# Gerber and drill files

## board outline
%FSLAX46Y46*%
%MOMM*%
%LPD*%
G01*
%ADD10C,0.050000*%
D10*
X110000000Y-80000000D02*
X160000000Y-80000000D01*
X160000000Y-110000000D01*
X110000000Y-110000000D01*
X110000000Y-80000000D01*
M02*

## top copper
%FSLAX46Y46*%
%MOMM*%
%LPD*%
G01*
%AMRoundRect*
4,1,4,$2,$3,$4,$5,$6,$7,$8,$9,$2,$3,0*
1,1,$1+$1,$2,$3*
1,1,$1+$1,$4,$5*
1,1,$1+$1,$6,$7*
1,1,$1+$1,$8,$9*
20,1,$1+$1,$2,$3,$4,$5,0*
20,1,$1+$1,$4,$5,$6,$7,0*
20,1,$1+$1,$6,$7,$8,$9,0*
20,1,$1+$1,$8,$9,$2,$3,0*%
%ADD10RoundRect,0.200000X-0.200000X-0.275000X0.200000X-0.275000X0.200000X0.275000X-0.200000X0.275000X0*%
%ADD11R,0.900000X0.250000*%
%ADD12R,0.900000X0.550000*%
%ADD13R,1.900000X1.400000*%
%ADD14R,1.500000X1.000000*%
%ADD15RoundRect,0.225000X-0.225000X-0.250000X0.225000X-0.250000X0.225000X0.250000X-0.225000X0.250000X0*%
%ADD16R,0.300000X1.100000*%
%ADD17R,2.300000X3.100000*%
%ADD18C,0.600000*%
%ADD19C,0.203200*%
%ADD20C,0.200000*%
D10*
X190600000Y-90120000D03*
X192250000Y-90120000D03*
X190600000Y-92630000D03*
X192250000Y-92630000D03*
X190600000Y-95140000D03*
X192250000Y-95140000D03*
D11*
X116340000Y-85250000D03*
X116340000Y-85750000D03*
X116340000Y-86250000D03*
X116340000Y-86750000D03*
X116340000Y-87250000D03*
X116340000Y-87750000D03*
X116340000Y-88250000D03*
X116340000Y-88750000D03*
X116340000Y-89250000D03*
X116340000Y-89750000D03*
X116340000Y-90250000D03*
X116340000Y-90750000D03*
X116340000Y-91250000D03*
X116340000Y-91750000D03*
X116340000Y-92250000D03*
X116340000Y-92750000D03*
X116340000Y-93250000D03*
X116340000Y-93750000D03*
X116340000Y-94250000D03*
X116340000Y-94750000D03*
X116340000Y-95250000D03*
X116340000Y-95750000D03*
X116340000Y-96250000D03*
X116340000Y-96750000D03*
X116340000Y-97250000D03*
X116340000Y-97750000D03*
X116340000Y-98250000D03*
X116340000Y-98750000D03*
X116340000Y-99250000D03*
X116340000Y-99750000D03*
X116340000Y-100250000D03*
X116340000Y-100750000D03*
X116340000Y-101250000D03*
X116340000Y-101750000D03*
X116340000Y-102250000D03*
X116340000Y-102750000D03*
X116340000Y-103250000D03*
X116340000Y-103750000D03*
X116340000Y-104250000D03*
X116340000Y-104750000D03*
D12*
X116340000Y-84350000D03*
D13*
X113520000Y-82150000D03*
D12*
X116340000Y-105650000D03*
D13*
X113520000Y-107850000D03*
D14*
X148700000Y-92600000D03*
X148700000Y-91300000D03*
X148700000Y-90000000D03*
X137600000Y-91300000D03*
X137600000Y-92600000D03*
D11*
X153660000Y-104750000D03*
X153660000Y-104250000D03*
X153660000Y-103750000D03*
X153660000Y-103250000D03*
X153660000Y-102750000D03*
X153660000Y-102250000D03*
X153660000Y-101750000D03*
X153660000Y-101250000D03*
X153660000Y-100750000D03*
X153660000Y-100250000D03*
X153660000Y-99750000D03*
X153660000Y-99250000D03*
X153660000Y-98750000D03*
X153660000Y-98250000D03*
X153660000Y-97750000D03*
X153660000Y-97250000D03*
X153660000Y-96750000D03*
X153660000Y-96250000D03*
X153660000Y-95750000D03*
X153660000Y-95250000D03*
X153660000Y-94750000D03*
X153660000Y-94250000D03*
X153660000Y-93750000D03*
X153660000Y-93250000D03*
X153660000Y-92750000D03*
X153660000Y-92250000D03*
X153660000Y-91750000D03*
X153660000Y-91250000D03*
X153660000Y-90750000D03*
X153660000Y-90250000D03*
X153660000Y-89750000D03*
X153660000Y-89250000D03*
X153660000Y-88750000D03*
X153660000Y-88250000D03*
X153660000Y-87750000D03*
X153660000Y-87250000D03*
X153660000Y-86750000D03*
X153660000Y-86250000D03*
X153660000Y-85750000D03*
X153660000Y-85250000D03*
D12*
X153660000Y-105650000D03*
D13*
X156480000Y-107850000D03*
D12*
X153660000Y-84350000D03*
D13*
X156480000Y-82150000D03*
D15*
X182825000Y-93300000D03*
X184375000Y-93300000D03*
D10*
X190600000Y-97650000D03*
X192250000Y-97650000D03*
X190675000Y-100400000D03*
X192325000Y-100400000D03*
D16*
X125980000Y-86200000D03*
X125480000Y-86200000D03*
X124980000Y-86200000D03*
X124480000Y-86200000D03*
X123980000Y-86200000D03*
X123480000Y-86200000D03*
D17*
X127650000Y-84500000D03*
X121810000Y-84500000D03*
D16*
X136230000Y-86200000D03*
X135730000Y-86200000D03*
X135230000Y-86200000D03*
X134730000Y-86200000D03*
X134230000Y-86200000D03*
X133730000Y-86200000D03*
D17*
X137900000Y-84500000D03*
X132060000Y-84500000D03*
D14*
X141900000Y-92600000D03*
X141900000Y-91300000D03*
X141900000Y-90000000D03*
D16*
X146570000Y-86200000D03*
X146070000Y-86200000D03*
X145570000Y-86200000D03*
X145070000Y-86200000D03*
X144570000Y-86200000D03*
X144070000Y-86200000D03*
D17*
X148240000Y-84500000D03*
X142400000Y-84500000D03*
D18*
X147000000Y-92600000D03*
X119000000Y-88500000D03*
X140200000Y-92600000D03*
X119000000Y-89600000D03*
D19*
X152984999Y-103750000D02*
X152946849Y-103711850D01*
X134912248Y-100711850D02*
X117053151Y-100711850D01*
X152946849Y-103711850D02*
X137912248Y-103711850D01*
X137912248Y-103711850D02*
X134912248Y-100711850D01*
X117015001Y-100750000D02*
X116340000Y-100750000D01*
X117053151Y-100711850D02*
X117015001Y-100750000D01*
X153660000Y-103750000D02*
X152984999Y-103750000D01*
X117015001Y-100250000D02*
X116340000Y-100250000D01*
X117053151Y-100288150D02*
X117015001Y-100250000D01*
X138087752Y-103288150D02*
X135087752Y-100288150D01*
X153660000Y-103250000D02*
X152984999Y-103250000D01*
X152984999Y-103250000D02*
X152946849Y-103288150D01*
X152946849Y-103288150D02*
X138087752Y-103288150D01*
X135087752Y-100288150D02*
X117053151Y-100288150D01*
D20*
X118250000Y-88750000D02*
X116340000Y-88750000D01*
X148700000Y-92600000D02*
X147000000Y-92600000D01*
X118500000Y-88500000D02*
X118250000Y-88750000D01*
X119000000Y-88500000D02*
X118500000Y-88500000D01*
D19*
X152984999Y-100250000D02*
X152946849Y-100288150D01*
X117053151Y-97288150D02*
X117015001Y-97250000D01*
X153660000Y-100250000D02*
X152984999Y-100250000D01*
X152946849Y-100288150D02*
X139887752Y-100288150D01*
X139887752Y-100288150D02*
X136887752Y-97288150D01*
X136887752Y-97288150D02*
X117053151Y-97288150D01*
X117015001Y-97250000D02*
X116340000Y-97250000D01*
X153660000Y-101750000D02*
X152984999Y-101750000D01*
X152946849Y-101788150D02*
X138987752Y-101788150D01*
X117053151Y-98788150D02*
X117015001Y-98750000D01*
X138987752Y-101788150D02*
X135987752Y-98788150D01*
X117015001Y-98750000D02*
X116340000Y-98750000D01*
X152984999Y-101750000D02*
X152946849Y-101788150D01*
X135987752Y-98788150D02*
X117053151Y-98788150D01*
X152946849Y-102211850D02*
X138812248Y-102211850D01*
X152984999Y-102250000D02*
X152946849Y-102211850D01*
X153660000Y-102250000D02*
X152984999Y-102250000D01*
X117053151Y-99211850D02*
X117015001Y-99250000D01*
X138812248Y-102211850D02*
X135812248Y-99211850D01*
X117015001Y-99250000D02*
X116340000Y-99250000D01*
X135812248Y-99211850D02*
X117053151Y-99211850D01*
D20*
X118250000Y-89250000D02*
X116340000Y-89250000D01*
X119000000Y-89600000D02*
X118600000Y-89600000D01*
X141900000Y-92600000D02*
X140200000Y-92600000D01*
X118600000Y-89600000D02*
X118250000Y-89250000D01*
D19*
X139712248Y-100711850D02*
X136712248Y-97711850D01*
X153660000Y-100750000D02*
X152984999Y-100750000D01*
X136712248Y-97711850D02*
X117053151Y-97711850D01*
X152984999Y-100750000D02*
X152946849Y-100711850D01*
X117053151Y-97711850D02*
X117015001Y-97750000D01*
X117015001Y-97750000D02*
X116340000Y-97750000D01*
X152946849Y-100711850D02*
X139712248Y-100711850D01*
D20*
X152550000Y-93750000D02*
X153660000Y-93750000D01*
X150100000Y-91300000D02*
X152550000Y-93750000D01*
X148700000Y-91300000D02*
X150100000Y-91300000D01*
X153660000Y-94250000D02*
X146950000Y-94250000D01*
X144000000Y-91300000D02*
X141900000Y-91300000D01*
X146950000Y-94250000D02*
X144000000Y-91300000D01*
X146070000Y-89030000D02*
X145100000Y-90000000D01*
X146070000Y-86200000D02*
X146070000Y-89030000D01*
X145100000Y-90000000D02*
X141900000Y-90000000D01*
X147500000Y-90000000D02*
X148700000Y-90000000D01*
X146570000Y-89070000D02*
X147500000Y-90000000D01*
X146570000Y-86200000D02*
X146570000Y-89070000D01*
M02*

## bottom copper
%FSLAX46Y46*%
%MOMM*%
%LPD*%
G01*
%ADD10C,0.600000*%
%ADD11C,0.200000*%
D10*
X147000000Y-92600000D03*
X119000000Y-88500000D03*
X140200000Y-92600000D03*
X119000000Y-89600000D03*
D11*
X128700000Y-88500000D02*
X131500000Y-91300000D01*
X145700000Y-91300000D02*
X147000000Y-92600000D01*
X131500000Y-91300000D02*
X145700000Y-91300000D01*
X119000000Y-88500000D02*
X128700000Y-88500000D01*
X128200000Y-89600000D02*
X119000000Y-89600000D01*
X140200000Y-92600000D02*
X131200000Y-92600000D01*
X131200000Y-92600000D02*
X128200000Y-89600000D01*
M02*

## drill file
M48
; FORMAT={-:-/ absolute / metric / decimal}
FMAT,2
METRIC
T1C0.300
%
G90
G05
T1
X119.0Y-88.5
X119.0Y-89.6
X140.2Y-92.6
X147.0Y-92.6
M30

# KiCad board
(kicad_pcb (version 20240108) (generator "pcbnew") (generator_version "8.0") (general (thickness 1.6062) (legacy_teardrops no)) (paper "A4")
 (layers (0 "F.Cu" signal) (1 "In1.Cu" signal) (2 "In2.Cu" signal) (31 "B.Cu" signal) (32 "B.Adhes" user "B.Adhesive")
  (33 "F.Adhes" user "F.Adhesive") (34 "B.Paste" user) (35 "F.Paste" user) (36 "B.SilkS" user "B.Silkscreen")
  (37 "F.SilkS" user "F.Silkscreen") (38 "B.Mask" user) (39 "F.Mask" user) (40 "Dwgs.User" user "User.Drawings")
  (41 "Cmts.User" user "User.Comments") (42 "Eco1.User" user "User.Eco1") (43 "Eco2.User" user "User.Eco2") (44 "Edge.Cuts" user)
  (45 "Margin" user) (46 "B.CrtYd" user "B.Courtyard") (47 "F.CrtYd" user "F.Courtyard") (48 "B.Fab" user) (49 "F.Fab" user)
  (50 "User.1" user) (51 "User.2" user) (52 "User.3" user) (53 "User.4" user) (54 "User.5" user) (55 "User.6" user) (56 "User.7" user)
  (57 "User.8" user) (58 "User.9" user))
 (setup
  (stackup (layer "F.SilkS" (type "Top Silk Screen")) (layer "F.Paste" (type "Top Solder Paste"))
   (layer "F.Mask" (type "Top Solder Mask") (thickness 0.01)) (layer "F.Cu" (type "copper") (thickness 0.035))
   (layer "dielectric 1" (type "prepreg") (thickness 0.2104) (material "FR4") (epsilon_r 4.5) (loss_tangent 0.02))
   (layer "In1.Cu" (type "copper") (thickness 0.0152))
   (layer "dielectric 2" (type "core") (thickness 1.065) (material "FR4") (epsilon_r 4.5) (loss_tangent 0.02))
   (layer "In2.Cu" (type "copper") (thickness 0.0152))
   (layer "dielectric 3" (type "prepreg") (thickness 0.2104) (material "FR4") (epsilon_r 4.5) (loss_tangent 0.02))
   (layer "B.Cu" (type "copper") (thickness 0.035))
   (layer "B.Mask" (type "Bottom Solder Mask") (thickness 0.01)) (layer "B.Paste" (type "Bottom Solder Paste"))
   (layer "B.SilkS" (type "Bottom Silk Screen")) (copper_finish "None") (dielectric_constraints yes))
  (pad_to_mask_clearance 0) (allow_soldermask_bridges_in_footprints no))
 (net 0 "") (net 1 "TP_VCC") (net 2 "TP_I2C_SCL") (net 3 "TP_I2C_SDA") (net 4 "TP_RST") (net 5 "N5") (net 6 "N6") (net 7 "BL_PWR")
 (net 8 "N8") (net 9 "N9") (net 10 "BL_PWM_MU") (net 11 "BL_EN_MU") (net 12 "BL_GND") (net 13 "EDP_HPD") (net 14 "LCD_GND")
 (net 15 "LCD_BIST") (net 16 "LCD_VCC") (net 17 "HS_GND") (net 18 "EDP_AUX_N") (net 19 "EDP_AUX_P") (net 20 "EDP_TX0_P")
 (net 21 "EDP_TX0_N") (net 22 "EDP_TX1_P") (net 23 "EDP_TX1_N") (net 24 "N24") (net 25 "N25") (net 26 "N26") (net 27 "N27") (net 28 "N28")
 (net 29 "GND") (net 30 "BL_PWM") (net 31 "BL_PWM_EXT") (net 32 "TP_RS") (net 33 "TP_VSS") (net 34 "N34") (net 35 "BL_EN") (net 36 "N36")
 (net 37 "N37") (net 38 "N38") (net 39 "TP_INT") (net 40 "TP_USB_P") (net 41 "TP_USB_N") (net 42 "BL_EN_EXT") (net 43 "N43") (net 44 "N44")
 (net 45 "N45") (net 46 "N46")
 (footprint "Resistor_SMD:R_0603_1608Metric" (layer "F.Cu") (at 191.425 90.12)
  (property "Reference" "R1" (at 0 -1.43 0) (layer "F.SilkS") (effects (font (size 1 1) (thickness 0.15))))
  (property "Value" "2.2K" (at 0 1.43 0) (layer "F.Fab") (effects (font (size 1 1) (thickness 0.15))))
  (pad "1" smd roundrect (at -0.825 0) (size 0.8 0.95) (layers "F.Cu" "F.Paste" "F.Mask") (roundrect_rratio 0.25) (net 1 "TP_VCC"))
  (pad "2" smd roundrect (at 0.825 0) (size 0.8 0.95) (layers "F.Cu" "F.Paste" "F.Mask") (roundrect_rratio 0.25) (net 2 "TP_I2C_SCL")))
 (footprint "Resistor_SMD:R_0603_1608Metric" (layer "F.Cu") (at 191.425 92.63)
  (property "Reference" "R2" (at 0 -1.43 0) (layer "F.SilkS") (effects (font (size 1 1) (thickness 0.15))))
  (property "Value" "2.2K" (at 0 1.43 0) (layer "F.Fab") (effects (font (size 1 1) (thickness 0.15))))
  (pad "1" smd roundrect (at -0.825 0) (size 0.8 0.95) (layers "F.Cu" "F.Paste" "F.Mask") (roundrect_rratio 0.25) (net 1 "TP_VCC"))
  (pad "2" smd roundrect (at 0.825 0) (size 0.8 0.95) (layers "F.Cu" "F.Paste" "F.Mask") (roundrect_rratio 0.25) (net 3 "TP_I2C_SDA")))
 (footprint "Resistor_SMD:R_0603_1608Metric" (layer "F.Cu") (at 191.425 95.14)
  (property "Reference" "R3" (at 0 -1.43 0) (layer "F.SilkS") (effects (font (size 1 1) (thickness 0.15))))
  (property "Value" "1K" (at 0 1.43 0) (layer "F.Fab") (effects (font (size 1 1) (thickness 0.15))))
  (pad "1" smd roundrect (at -0.825 0) (size 0.8 0.95) (layers "F.Cu" "F.Paste" "F.Mask") (roundrect_rratio 0.25) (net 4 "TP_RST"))
  (pad "2" smd roundrect (at 0.825 0) (size 0.8 0.95) (layers "F.Cu" "F.Paste" "F.Mask") (roundrect_rratio 0.25) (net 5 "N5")))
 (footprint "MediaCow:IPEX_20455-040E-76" (layer "F.Cu") (at 114.42 95 -90)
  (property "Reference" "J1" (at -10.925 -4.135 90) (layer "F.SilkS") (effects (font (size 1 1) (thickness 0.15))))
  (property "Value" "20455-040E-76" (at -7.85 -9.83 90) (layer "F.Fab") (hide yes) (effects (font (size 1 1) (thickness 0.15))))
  (pad "1" smd rect (at -9.75 -1.92 270) (size 0.25 0.9) (layers "F.Cu" "F.Paste" "F.Mask") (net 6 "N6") (solder_mask_margin 0.102))
  (pad "2" smd rect (at -9.25 -1.92 270) (size 0.25 0.9) (layers "F.Cu" "F.Paste" "F.Mask") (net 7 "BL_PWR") (solder_mask_margin 0.102))
  (pad "3" smd rect (at -8.75 -1.92 270) (size 0.25 0.9) (layers "F.Cu" "F.Paste" "F.Mask") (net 7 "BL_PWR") (solder_mask_margin 0.102))
  (pad "4" smd rect (at -8.25 -1.92 270) (size 0.25 0.9) (layers "F.Cu" "F.Paste" "F.Mask") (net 7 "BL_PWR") (solder_mask_margin 0.102))
  (pad "5" smd rect (at -7.75 -1.92 270) (size 0.25 0.9) (layers "F.Cu" "F.Paste" "F.Mask") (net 7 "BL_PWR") (solder_mask_margin 0.102))
  (pad "6" smd rect (at -7.25 -1.92 270) (size 0.25 0.9) (layers "F.Cu" "F.Paste" "F.Mask") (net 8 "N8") (solder_mask_margin 0.102))
  (pad "7" smd rect (at -6.75 -1.92 270) (size 0.25 0.9) (layers "F.Cu" "F.Paste" "F.Mask") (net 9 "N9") (solder_mask_margin 0.102))
  (pad "8" smd rect (at -6.25 -1.92 270) (size 0.25 0.9) (layers "F.Cu" "F.Paste" "F.Mask") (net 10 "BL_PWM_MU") (solder_mask_margin 0.102))
  (pad "9" smd rect (at -5.75 -1.92 270) (size 0.25 0.9) (layers "F.Cu" "F.Paste" "F.Mask") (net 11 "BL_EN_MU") (solder_mask_margin 0.102))
  (pad "10" smd rect (at -5.25 -1.92 270) (size 0.25 0.9) (layers "F.Cu" "F.Paste" "F.Mask") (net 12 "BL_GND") (solder_mask_margin 0.102))
  (pad "11" smd rect (at -4.75 -1.92 270) (size 0.25 0.9) (layers "F.Cu" "F.Paste" "F.Mask") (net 12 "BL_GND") (solder_mask_margin 0.102))
  (pad "12" smd rect (at -4.25 -1.92 270) (size 0.25 0.9) (layers "F.Cu" "F.Paste" "F.Mask") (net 12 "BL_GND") (solder_mask_margin 0.102))
  (pad "13" smd rect (at -3.75 -1.92 270) (size 0.25 0.9) (layers "F.Cu" "F.Paste" "F.Mask") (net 12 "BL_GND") (solder_mask_margin 0.102))
  (pad "14" smd rect (at -3.25 -1.92 270) (size 0.25 0.9) (layers "F.Cu" "F.Paste" "F.Mask") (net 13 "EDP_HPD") (solder_mask_margin 0.102))
  (pad "15" smd rect (at -2.75 -1.92 270) (size 0.25 0.9) (layers "F.Cu" "F.Paste" "F.Mask") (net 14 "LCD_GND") (solder_mask_margin 0.102))
  (pad "16" smd rect (at -2.25 -1.92 270) (size 0.25 0.9) (layers "F.Cu" "F.Paste" "F.Mask") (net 14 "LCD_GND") (solder_mask_margin 0.102))
  (pad "17" smd rect (at -1.75 -1.92 270) (size 0.25 0.9) (layers "F.Cu" "F.Paste" "F.Mask") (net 14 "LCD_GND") (solder_mask_margin 0.102))
  (pad "18" smd rect (at -1.25 -1.92 270) (size 0.25 0.9) (layers "F.Cu" "F.Paste" "F.Mask") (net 14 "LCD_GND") (solder_mask_margin 0.102))
  (pad "19" smd rect (at -0.75 -1.92 270) (size 0.25 0.9) (layers "F.Cu" "F.Paste" "F.Mask") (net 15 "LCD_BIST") (solder_mask_margin 0.102))
  (pad "20" smd rect (at -0.25 -1.92 270) (size 0.25 0.9) (layers "F.Cu" "F.Paste" "F.Mask") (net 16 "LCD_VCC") (solder_mask_margin 0.102))
  (pad "21" smd rect (at 0.25 -1.92 270) (size 0.25 0.9) (layers "F.Cu" "F.Paste" "F.Mask") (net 16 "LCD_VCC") (solder_mask_margin 0.102))
  (pad "22" smd rect (at 0.75 -1.92 270) (size 0.25 0.9) (layers "F.Cu" "F.Paste" "F.Mask") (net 16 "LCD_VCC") (solder_mask_margin 0.102))
  (pad "23" smd rect (at 1.25 -1.92 270) (size 0.25 0.9) (layers "F.Cu" "F.Paste" "F.Mask") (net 16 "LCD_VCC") (solder_mask_margin 0.102))
  (pad "24" smd rect (at 1.75 -1.92 270) (size 0.25 0.9) (layers "F.Cu" "F.Paste" "F.Mask") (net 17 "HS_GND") (solder_mask_margin 0.102))
  (pad "25" smd rect (at 2.25 -1.92 270) (size 0.25 0.9) (layers "F.Cu" "F.Paste" "F.Mask") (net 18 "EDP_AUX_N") (solder_mask_margin 0.102))
  (pad "26" smd rect (at 2.75 -1.92 270) (size 0.25 0.9) (layers "F.Cu" "F.Paste" "F.Mask") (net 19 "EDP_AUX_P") (solder_mask_margin 0.102))
  (pad "27" smd rect (at 3.25 -1.92 270) (size 0.25 0.9) (layers "F.Cu" "F.Paste" "F.Mask") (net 17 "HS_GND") (solder_mask_margin 0.102))
  (pad "28" smd rect (at 3.75 -1.92 270) (size 0.25 0.9) (layers "F.Cu" "F.Paste" "F.Mask") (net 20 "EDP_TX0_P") (solder_mask_margin 0.102))
  (pad "29" smd rect (at 4.25 -1.92 270) (size 0.25 0.9) (layers "F.Cu" "F.Paste" "F.Mask") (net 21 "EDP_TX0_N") (solder_mask_margin 0.102))
  (pad "30" smd rect (at 4.75 -1.92 270) (size 0.25 0.9) (layers "F.Cu" "F.Paste" "F.Mask") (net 17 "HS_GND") (solder_mask_margin 0.102))
  (pad "31" smd rect (at 5.25 -1.92 270) (size 0.25 0.9) (layers "F.Cu" "F.Paste" "F.Mask") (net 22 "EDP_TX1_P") (solder_mask_margin 0.102))
  (pad "32" smd rect (at 5.75 -1.92 270) (size 0.25 0.9) (layers "F.Cu" "F.Paste" "F.Mask") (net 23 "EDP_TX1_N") (solder_mask_margin 0.102))
  (pad "33" smd rect (at 6.25 -1.92 270) (size 0.25 0.9) (layers "F.Cu" "F.Paste" "F.Mask") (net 17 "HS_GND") (solder_mask_margin 0.102))
  (pad "34" smd rect (at 6.75 -1.92 270) (size 0.25 0.9) (layers "F.Cu" "F.Paste" "F.Mask") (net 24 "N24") (solder_mask_margin 0.102))
  (pad "35" smd rect (at 7.25 -1.92 270) (size 0.25 0.9) (layers "F.Cu" "F.Paste" "F.Mask") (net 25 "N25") (solder_mask_margin 0.102))
  (pad "36" smd rect (at 7.75 -1.92 270) (size 0.25 0.9) (layers "F.Cu" "F.Paste" "F.Mask") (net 17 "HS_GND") (solder_mask_margin 0.102))
  (pad "37" smd rect (at 8.25 -1.92 270) (size 0.25 0.9) (layers "F.Cu" "F.Paste" "F.Mask") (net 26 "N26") (solder_mask_margin 0.102))
  (pad "38" smd rect (at 8.75 -1.92 270) (size 0.25 0.9) (layers "F.Cu" "F.Paste" "F.Mask") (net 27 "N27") (solder_mask_margin 0.102))
  (pad "39" smd rect (at 9.25 -1.92 270) (size 0.25 0.9) (layers "F.Cu" "F.Paste" "F.Mask") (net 17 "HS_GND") (solder_mask_margin 0.102))
  (pad "40" smd rect (at 9.75 -1.92 270) (size 0.25 0.9) (layers "F.Cu" "F.Paste" "F.Mask") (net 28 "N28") (solder_mask_margin 0.102))
  (pad "S1" smd rect (at -10.65 -1.92 270) (size 0.55 0.9) (layers "F.Cu" "F.Paste" "F.Mask") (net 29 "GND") (solder_mask_margin 0.102))
  (pad "S2" smd rect (at -12.85 0.9 270) (size 1.4 1.9) (layers "F.Cu" "F.Paste" "F.Mask") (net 29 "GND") (solder_mask_margin 0.102))
  (pad "S3" smd rect (at 10.65 -1.92 270) (size 0.55 0.9) (layers "F.Cu" "F.Paste" "F.Mask") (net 29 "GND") (solder_mask_margin 0.102))
  (pad "S4" smd rect (at 12.85 0.9 270) (size 1.4 1.9) (layers "F.Cu" "F.Paste" "F.Mask") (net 29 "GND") (solder_mask_margin 0.102)))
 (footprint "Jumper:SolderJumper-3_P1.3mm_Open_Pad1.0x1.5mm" (layer "F.Cu") (at 148.7 91.3 90)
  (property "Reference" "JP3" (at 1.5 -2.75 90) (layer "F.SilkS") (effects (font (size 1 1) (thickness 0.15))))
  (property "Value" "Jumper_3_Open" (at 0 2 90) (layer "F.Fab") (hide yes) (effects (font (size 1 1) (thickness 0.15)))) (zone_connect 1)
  (pad "1" smd rect (at -1.3 0 90) (size 1 1.5) (layers "F.Cu" "F.Mask") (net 10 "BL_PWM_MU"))
  (pad "2" smd rect (at 0 0 90) (size 1 1.5) (layers "F.Cu" "F.Mask") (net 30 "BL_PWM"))
  (pad "3" smd rect (at 1.3 0 90) (size 1 1.5) (layers "F.Cu" "F.Mask") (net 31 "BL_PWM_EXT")))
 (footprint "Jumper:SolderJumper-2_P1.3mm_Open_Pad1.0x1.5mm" (layer "F.Cu") (at 137.6 91.95 -90)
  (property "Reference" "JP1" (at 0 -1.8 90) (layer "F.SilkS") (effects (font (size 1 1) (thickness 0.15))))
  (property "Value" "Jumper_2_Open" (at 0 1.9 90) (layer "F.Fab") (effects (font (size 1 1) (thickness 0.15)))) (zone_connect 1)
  (pad "1" smd rect (at -0.65 0 270) (size 1 1.5) (layers "F.Cu" "F.Mask") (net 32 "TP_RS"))
  (pad "2" smd rect (at 0.65 0 270) (size 1 1.5) (layers "F.Cu" "F.Mask") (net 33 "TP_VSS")))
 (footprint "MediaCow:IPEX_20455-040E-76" (layer "F.Cu") (at 155.58 95 90)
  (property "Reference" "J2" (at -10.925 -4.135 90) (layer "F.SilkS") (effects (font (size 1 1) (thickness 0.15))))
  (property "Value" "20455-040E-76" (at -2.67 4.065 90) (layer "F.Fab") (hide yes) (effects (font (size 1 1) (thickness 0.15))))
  (pad "1" smd rect (at -9.75 -1.92 90) (size 0.25 0.9) (layers "F.Cu" "F.Paste" "F.Mask") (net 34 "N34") (solder_mask_margin 0.102))
  (pad "2" smd rect (at -9.25 -1.92 90) (size 0.25 0.9) (layers "F.Cu" "F.Paste" "F.Mask") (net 17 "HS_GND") (solder_mask_margin 0.102))
  (pad "3" smd rect (at -8.75 -1.92 90) (size 0.25 0.9) (layers "F.Cu" "F.Paste" "F.Mask") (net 23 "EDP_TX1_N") (solder_mask_margin 0.102))
  (pad "4" smd rect (at -8.25 -1.92 90) (size 0.25 0.9) (layers "F.Cu" "F.Paste" "F.Mask") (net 22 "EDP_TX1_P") (solder_mask_margin 0.102))
  (pad "5" smd rect (at -7.75 -1.92 90) (size 0.25 0.9) (layers "F.Cu" "F.Paste" "F.Mask") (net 17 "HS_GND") (solder_mask_margin 0.102))
  (pad "6" smd rect (at -7.25 -1.92 90) (size 0.25 0.9) (layers "F.Cu" "F.Paste" "F.Mask") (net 21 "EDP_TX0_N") (solder_mask_margin 0.102))
  (pad "7" smd rect (at -6.75 -1.92 90) (size 0.25 0.9) (layers "F.Cu" "F.Paste" "F.Mask") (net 20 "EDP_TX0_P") (solder_mask_margin 0.102))
  (pad "8" smd rect (at -6.25 -1.92 90) (size 0.25 0.9) (layers "F.Cu" "F.Paste" "F.Mask") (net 17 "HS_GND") (solder_mask_margin 0.102))
  (pad "9" smd rect (at -5.75 -1.92 90) (size 0.25 0.9) (layers "F.Cu" "F.Paste" "F.Mask") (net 19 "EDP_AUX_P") (solder_mask_margin 0.102))
  (pad "10" smd rect (at -5.25 -1.92 90) (size 0.25 0.9) (layers "F.Cu" "F.Paste" "F.Mask") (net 18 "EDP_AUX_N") (solder_mask_margin 0.102))
  (pad "11" smd rect (at -4.75 -1.92 90) (size 0.25 0.9) (layers "F.Cu" "F.Paste" "F.Mask") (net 17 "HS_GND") (solder_mask_margin 0.102))
  (pad "12" smd rect (at -4.25 -1.92 90) (size 0.25 0.9) (layers "F.Cu" "F.Paste" "F.Mask") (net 16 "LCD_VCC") (solder_mask_margin 0.102))
  (pad "13" smd rect (at -3.75 -1.92 90) (size 0.25 0.9) (layers "F.Cu" "F.Paste" "F.Mask") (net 16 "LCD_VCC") (solder_mask_margin 0.102))
  (pad "14" smd rect (at -3.25 -1.92 90) (size 0.25 0.9) (layers "F.Cu" "F.Paste" "F.Mask") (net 15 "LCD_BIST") (solder_mask_margin 0.102))
  (pad "15" smd rect (at -2.75 -1.92 90) (size 0.25 0.9) (layers "F.Cu" "F.Paste" "F.Mask") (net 14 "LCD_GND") (solder_mask_margin 0.102))
  (pad "16" smd rect (at -2.25 -1.92 90) (size 0.25 0.9) (layers "F.Cu" "F.Paste" "F.Mask") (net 14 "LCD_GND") (solder_mask_margin 0.102))
  (pad "17" smd rect (at -1.75 -1.92 90) (size 0.25 0.9) (layers "F.Cu" "F.Paste" "F.Mask") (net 13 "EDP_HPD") (solder_mask_margin 0.102))
  (pad "18" smd rect (at -1.25 -1.92 90) (size 0.25 0.9) (layers "F.Cu" "F.Paste" "F.Mask") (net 12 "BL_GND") (solder_mask_margin 0.102))
  (pad "19" smd rect (at -0.75 -1.92 90) (size 0.25 0.9) (layers "F.Cu" "F.Paste" "F.Mask") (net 12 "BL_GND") (solder_mask_margin 0.102))
  (pad "20" smd rect (at -0.25 -1.92 90) (size 0.25 0.9) (layers "F.Cu" "F.Paste" "F.Mask") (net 12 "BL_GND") (solder_mask_margin 0.102))
  (pad "21" smd rect (at 0.25 -1.92 90) (size 0.25 0.9) (layers "F.Cu" "F.Paste" "F.Mask") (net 12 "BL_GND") (solder_mask_margin 0.102))
  (pad "22" smd rect (at 0.75 -1.92 90) (size 0.25 0.9) (layers "F.Cu" "F.Paste" "F.Mask") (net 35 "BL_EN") (solder_mask_margin 0.102))
  (pad "23" smd rect (at 1.25 -1.92 90) (size 0.25 0.9) (layers "F.Cu" "F.Paste" "F.Mask") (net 30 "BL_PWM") (solder_mask_margin 0.102))
  (pad "24" smd rect (at 1.75 -1.92 90) (size 0.25 0.9) (layers "F.Cu" "F.Paste" "F.Mask") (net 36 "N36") (solder_mask_margin 0.102))
  (pad "25" smd rect (at 2.25 -1.92 90) (size 0.25 0.9) (layers "F.Cu" "F.Paste" "F.Mask") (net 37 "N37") (solder_mask_margin 0.102))
  (pad "26" smd rect (at 2.75 -1.92 90) (size 0.25 0.9) (layers "F.Cu" "F.Paste" "F.Mask") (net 7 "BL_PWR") (solder_mask_margin 0.102))
  (pad "27" smd rect (at 3.25 -1.92 90) (size 0.25 0.9) (layers "F.Cu" "F.Paste" "F.Mask") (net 7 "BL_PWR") (solder_mask_margin 0.102))
  (pad "28" smd rect (at 3.75 -1.92 90) (size 0.25 0.9) (layers "F.Cu" "F.Paste" "F.Mask") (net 7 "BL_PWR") (solder_mask_margin 0.102))
  (pad "29" smd rect (at 4.25 -1.92 90) (size 0.25 0.9) (layers "F.Cu" "F.Paste" "F.Mask") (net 7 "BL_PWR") (solder_mask_margin 0.102))
  (pad "30" smd rect (at 4.75 -1.92 90) (size 0.25 0.9) (layers "F.Cu" "F.Paste" "F.Mask") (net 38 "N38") (solder_mask_margin 0.102))
  (pad "31" smd rect (at 5.25 -1.92 90) (size 0.25 0.9) (layers "F.Cu" "F.Paste" "F.Mask") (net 4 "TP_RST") (solder_mask_margin 0.102))
  (pad "32" smd rect (at 5.75 -1.92 90) (size 0.25 0.9) (layers "F.Cu" "F.Paste" "F.Mask") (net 2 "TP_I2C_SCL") (solder_mask_margin 0.102))
  (pad "33" smd rect (at 6.25 -1.92 90) (size 0.25 0.9) (layers "F.Cu" "F.Paste" "F.Mask") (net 3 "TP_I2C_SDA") (solder_mask_margin 0.102))
  (pad "34" smd rect (at 6.75 -1.92 90) (size 0.25 0.9) (layers "F.Cu" "F.Paste" "F.Mask") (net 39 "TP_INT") (solder_mask_margin 0.102))
  (pad "35" smd rect (at 7.25 -1.92 90) (size 0.25 0.9) (layers "F.Cu" "F.Paste" "F.Mask") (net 33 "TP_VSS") (solder_mask_margin 0.102))
  (pad "36" smd rect (at 7.75 -1.92 90) (size 0.25 0.9) (layers "F.Cu" "F.Paste" "F.Mask") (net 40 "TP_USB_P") (solder_mask_margin 0.102))
  (pad "37" smd rect (at 8.25 -1.92 90) (size 0.25 0.9) (layers "F.Cu" "F.Paste" "F.Mask") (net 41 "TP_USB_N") (solder_mask_margin 0.102))
  (pad "38" smd rect (at 8.75 -1.92 90) (size 0.25 0.9) (layers "F.Cu" "F.Paste" "F.Mask") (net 33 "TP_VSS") (solder_mask_margin 0.102))
  (pad "39" smd rect (at 9.25 -1.92 90) (size 0.25 0.9) (layers "F.Cu" "F.Paste" "F.Mask") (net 32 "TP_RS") (solder_mask_margin 0.102))
  (pad "40" smd rect (at 9.75 -1.92 90) (size 0.25 0.9) (layers "F.Cu" "F.Paste" "F.Mask") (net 1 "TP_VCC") (solder_mask_margin 0.102))
  (pad "S1" smd rect (at -10.65 -1.92 90) (size 0.55 0.9) (layers "F.Cu" "F.Paste" "F.Mask") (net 29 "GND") (solder_mask_margin 0.102))
  (pad "S2" smd rect (at -12.85 0.9 90) (size 1.4 1.9) (layers "F.Cu" "F.Paste" "F.Mask") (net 29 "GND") (solder_mask_margin 0.102))
  (pad "S3" smd rect (at 10.65 -1.92 90) (size 0.55 0.9) (layers "F.Cu" "F.Paste" "F.Mask") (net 29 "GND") (solder_mask_margin 0.102))
  (pad "S4" smd rect (at 12.85 0.9 90) (size 1.4 1.9) (layers "F.Cu" "F.Paste" "F.Mask") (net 29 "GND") (solder_mask_margin 0.102)))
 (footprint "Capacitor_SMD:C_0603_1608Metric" (layer "F.Cu") (at 183.6 93.3)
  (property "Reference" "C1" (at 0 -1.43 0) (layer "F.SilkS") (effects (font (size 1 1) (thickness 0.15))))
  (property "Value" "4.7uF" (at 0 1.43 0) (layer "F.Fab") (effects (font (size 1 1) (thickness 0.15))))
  (pad "1" smd roundrect (at -0.775 0) (size 0.9 0.95) (layers "F.Cu" "F.Paste" "F.Mask") (roundrect_rratio 0.25) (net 5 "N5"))
  (pad "2" smd roundrect (at 0.775 0) (size 0.9 0.95) (layers "F.Cu" "F.Paste" "F.Mask") (roundrect_rratio 0.25) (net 33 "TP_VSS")))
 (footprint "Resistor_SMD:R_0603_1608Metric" (layer "F.Cu") (at 191.425 97.65)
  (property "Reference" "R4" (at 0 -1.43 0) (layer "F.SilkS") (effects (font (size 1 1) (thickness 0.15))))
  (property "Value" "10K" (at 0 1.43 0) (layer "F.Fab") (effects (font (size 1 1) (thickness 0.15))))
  (pad "1" smd roundrect (at -0.825 0) (size 0.8 0.95) (layers "F.Cu" "F.Paste" "F.Mask") (roundrect_rratio 0.25) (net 1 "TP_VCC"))
  (pad "2" smd roundrect (at 0.825 0) (size 0.8 0.95) (layers "F.Cu" "F.Paste" "F.Mask") (roundrect_rratio 0.25) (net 5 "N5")))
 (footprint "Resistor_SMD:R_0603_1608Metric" (layer "F.Cu") (at 191.5 100.4)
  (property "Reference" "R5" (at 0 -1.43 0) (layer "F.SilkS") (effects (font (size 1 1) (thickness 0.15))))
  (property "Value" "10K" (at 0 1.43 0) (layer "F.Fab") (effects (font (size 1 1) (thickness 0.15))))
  (pad "1" smd roundrect (at -0.825 0) (size 0.8 0.95) (layers "F.Cu" "F.Paste" "F.Mask") (roundrect_rratio 0.25) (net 1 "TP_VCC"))
  (pad "2" smd roundrect (at 0.825 0) (size 0.8 0.95) (layers "F.Cu" "F.Paste" "F.Mask") (roundrect_rratio 0.25) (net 32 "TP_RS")))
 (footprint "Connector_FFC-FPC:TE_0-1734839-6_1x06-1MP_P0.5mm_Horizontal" (layer "F.Cu") (at 124.73 84.85 180)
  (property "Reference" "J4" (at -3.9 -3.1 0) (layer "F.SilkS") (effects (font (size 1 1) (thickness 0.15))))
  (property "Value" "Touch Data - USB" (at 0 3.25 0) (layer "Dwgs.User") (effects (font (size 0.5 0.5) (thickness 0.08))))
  (pad "1" smd rect (at -1.25 -1.35 180) (size 0.3 1.1) (layers "F.Cu" "F.Paste" "F.Mask") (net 33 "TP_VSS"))
  (pad "2" smd rect (at -0.75 -1.35 180) (size 0.3 1.1) (layers "F.Cu" "F.Paste" "F.Mask") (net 40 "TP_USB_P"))
  (pad "3" smd rect (at -0.25 -1.35 180) (size 0.3 1.1) (layers "F.Cu" "F.Paste" "F.Mask") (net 41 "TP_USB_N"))
  (pad "4" smd rect (at 0.25 -1.35 180) (size 0.3 1.1) (layers "F.Cu" "F.Paste" "F.Mask") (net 33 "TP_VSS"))
  (pad "5" smd rect (at 0.75 -1.35 180) (size 0.3 1.1) (layers "F.Cu" "F.Paste" "F.Mask") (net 4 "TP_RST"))
  (pad "6" smd rect (at 1.25 -1.35 180) (size 0.3 1.1) (layers "F.Cu" "F.Paste" "F.Mask") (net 1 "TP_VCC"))
  (pad "MP" smd rect (at -2.92 0.35 180) (size 2.3 3.1) (layers "F.Cu" "F.Paste" "F.Mask"))
  (pad "MP" smd rect (at 2.92 0.35 180) (size 2.3 3.1) (layers "F.Cu" "F.Paste" "F.Mask")))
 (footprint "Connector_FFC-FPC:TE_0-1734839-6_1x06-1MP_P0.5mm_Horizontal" (layer "F.Cu") (at 134.98 84.85 180)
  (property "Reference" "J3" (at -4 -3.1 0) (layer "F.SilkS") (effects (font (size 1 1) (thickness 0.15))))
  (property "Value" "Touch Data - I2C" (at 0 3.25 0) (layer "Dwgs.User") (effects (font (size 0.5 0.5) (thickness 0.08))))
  (pad "1" smd rect (at -1.25 -1.35 180) (size 0.3 1.1) (layers "F.Cu" "F.Paste" "F.Mask") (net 2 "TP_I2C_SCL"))
  (pad "2" smd rect (at -0.75 -1.35 180) (size 0.3 1.1) (layers "F.Cu" "F.Paste" "F.Mask") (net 3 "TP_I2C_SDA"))
  (pad "3" smd rect (at -0.25 -1.35 180) (size 0.3 1.1) (layers "F.Cu" "F.Paste" "F.Mask") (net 33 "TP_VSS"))
  (pad "4" smd rect (at 0.25 -1.35 180) (size 0.3 1.1) (layers "F.Cu" "F.Paste" "F.Mask") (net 4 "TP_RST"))
  (pad "5" smd rect (at 0.75 -1.35 180) (size 0.3 1.1) (layers "F.Cu" "F.Paste" "F.Mask") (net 39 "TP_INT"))
  (pad "6" smd rect (at 1.25 -1.35 180) (size 0.3 1.1) (layers "F.Cu" "F.Paste" "F.Mask") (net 1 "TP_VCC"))
  (pad "MP" smd rect (at -2.92 0.35 180) (size 2.3 3.1) (layers "F.Cu" "F.Paste" "F.Mask"))
  (pad "MP" smd rect (at 2.92 0.35 180) (size 2.3 3.1) (layers "F.Cu" "F.Paste" "F.Mask")))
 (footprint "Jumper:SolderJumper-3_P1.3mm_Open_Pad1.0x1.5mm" (layer "F.Cu") (at 141.9 91.3 90)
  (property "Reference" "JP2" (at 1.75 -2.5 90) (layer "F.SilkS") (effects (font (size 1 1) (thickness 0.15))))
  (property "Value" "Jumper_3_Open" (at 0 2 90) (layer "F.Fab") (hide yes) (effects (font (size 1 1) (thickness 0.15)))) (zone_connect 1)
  (pad "1" smd rect (at -1.3 0 90) (size 1 1.5) (layers "F.Cu" "F.Mask") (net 11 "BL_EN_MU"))
  (pad "2" smd rect (at 0 0 90) (size 1 1.5) (layers "F.Cu" "F.Mask") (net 35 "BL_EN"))
  (pad "3" smd rect (at 1.3 0 90) (size 1 1.5) (layers "F.Cu" "F.Mask") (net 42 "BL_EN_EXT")))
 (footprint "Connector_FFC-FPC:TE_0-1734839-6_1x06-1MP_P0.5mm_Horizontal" (layer "F.Cu") (at 145.32 84.85 180)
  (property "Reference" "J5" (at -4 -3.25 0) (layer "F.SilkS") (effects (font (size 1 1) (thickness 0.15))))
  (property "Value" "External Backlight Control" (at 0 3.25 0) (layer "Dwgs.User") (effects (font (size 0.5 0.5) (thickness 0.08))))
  (pad "1" smd rect (at -1.25 -1.35 180) (size 0.3 1.1) (layers "F.Cu" "F.Paste" "F.Mask") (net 31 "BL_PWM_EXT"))
  (pad "2" smd rect (at -0.75 -1.35 180) (size 0.3 1.1) (layers "F.Cu" "F.Paste" "F.Mask") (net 42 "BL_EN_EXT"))
  (pad "3" smd rect (at -0.25 -1.35 180) (size 0.3 1.1) (layers "F.Cu" "F.Paste" "F.Mask") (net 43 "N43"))
  (pad "4" smd rect (at 0.25 -1.35 180) (size 0.3 1.1) (layers "F.Cu" "F.Paste" "F.Mask") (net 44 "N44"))
  (pad "5" smd rect (at 0.75 -1.35 180) (size 0.3 1.1) (layers "F.Cu" "F.Paste" "F.Mask") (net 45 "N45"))
  (pad "6" smd rect (at 1.25 -1.35 180) (size 0.3 1.1) (layers "F.Cu" "F.Paste" "F.Mask") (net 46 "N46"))
  (pad "MP" smd rect (at -2.92 0.35 180) (size 2.3 3.1) (layers "F.Cu" "F.Paste" "F.Mask"))
  (pad "MP" smd rect (at 2.92 0.35 180) (size 2.3 3.1) (layers "F.Cu" "F.Paste" "F.Mask")))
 (gr_rect (start 110 80) (end 160 110) (stroke (width 0.05) (type default)) (fill none) (layer "Edge.Cuts"))
 (segment (start 152.984999 103.75) (end 152.946849 103.71185) (width 0.2032) (layer "F.Cu") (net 23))
 (segment (start 134.912248 100.71185) (end 117.053151 100.71185) (width 0.2032) (layer "F.Cu") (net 23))
 (segment (start 152.946849 103.71185) (end 137.912248 103.71185) (width 0.2032) (layer "F.Cu") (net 23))
 (segment (start 137.912248 103.71185) (end 134.912248 100.71185) (width 0.2032) (layer "F.Cu") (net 23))
 (segment (start 117.015001 100.75) (end 116.34 100.75) (width 0.2032) (layer "F.Cu") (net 23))
 (segment (start 117.053151 100.71185) (end 117.015001 100.75) (width 0.2032) (layer "F.Cu") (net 23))
 (segment (start 153.66 103.75) (end 152.984999 103.75) (width 0.2032) (layer "F.Cu") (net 23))
 (segment (start 117.015001 100.25) (end 116.34 100.25) (width 0.2032) (layer "F.Cu") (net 22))
 (segment (start 117.053151 100.28815) (end 117.015001 100.25) (width 0.2032) (layer "F.Cu") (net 22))
 (segment (start 138.087752 103.28815) (end 135.087752 100.28815) (width 0.2032) (layer "F.Cu") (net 22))
 (segment (start 153.66 103.25) (end 152.984999 103.25) (width 0.2032) (layer "F.Cu") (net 22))
 (segment (start 152.984999 103.25) (end 152.946849 103.28815) (width 0.2032) (layer "F.Cu") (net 22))
 (segment (start 152.946849 103.28815) (end 138.087752 103.28815) (width 0.2032) (layer "F.Cu") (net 22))
 (segment (start 135.087752 100.28815) (end 117.053151 100.28815) (width 0.2032) (layer "F.Cu") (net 22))
 (segment (start 118.25 88.75) (end 116.34 88.75) (width 0.2) (layer "F.Cu") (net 10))
 (segment (start 148.7 92.6) (end 147 92.6) (width 0.2) (layer "F.Cu") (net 10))
 (segment (start 118.5 88.5) (end 118.25 88.75) (width 0.2) (layer "F.Cu") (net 10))
 (segment (start 119 88.5) (end 118.5 88.5) (width 0.2) (layer "F.Cu") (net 10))
 (via (at 147 92.6) (size 0.6) (drill 0.3) (layers "F.Cu" "B.Cu") (free yes) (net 10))
 (via (at 119 88.5) (size 0.6) (drill 0.3) (layers "F.Cu" "B.Cu") (free yes) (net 10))
 (segment (start 128.7 88.5) (end 131.5 91.3) (width 0.2) (layer "B.Cu") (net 10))
 (segment (start 145.7 91.3) (end 147 92.6) (width 0.2) (layer "B.Cu") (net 10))
 (segment (start 131.5 91.3) (end 145.7 91.3) (width 0.2) (layer "B.Cu") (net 10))
 (segment (start 119 88.5) (end 128.7 88.5) (width 0.2) (layer "B.Cu") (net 10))
 (segment (start 152.984999 100.25) (end 152.946849 100.28815) (width 0.2032) (layer "F.Cu") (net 18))
 (segment (start 117.053151 97.28815) (end 117.015001 97.25) (width 0.2032) (layer "F.Cu") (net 18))
 (segment (start 153.66 100.25) (end 152.984999 100.25) (width 0.2032) (layer "F.Cu") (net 18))
 (segment (start 152.946849 100.28815) (end 139.887752 100.28815) (width 0.2032) (layer "F.Cu") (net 18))
 (segment (start 139.887752 100.28815) (end 136.887752 97.28815) (width 0.2032) (layer "F.Cu") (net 18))
 (segment (start 136.887752 97.28815) (end 117.053151 97.28815) (width 0.2032) (layer "F.Cu") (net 18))
 (segment (start 117.015001 97.25) (end 116.34 97.25) (width 0.2032) (layer "F.Cu") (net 18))
 (segment (start 153.66 101.75) (end 152.984999 101.75) (width 0.2032) (layer "F.Cu") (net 20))
 (segment (start 152.946849 101.78815) (end 138.987752 101.78815) (width 0.2032) (layer "F.Cu") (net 20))
 (segment (start 117.053151 98.78815) (end 117.015001 98.75) (width 0.2032) (layer "F.Cu") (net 20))
 (segment (start 138.987752 101.78815) (end 135.987752 98.78815) (width 0.2032) (layer "F.Cu") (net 20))
 (segment (start 117.015001 98.75) (end 116.34 98.75) (width 0.2032) (layer "F.Cu") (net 20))
 (segment (start 152.984999 101.75) (end 152.946849 101.78815) (width 0.2032) (layer "F.Cu") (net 20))
 (segment (start 135.987752 98.78815) (end 117.053151 98.78815) (width 0.2032) (layer "F.Cu") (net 20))
 (segment (start 152.946849 102.21185) (end 138.812248 102.21185) (width 0.2032) (layer "F.Cu") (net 21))
 (segment (start 152.984999 102.25) (end 152.946849 102.21185) (width 0.2032) (layer "F.Cu") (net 21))
 (segment (start 153.66 102.25) (end 152.984999 102.25) (width 0.2032) (layer "F.Cu") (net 21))
 (segment (start 117.053151 99.21185) (end 117.015001 99.25) (width 0.2032) (layer "F.Cu") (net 21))
 (segment (start 138.812248 102.21185) (end 135.812248 99.21185) (width 0.2032) (layer "F.Cu") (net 21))
 (segment (start 117.015001 99.25) (end 116.34 99.25) (width 0.2032) (layer "F.Cu") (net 21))
 (segment (start 135.812248 99.21185) (end 117.053151 99.21185) (width 0.2032) (layer "F.Cu") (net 21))
 (segment (start 118.25 89.25) (end 116.34 89.25) (width 0.2) (layer "F.Cu") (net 11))
 (segment (start 119 89.6) (end 118.6 89.6) (width 0.2) (layer "F.Cu") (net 11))
 (segment (start 141.9 92.6) (end 140.2 92.6) (width 0.2) (layer "F.Cu") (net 11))
 (segment (start 118.6 89.6) (end 118.25 89.25) (width 0.2) (layer "F.Cu") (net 11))
 (via (at 140.2 92.6) (size 0.6) (drill 0.3) (layers "F.Cu" "B.Cu") (free yes) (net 11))
 (via (at 119 89.6) (size 0.6) (drill 0.3) (layers "F.Cu" "B.Cu") (free yes) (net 11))
 (segment (start 128.2 89.6) (end 119 89.6) (width 0.2) (layer "B.Cu") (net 11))
 (segment (start 140.2 92.6) (end 131.2 92.6) (width 0.2) (layer "B.Cu") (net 11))
 (segment (start 131.2 92.6) (end 128.2 89.6) (width 0.2) (layer "B.Cu") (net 11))
 (segment (start 139.712248 100.71185) (end 136.712248 97.71185) (width 0.2032) (layer "F.Cu") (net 19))
 (segment (start 153.66 100.75) (end 152.984999 100.75) (width 0.2032) (layer "F.Cu") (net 19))
 (segment (start 136.712248 97.71185) (end 117.053151 97.71185) (width 0.2032) (layer "F.Cu") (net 19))
 (segment (start 152.984999 100.75) (end 152.946849 100.71185) (width 0.2032) (layer "F.Cu") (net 19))
 (segment (start 117.053151 97.71185) (end 117.015001 97.75) (width 0.2032) (layer "F.Cu") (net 19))
 (segment (start 117.015001 97.75) (end 116.34 97.75) (width 0.2032) (layer "F.Cu") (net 19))
 (segment (start 152.946849 100.71185) (end 139.712248 100.71185) (width 0.2032) (layer "F.Cu") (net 19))
 (segment (start 152.55 93.75) (end 153.66 93.75) (width 0.2) (layer "F.Cu") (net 30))
 (segment (start 150.1 91.3) (end 152.55 93.75) (width 0.2) (layer "F.Cu") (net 30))
 (segment (start 148.7 91.3) (end 150.1 91.3) (width 0.2) (layer "F.Cu") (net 30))
 (segment (start 153.66 94.25) (end 146.95 94.25) (width 0.2) (layer "F.Cu") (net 35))
 (segment (start 144 91.3) (end 141.9 91.3) (width 0.2) (layer "F.Cu") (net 35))
 (segment (start 146.95 94.25) (end 144 91.3) (width 0.2) (layer "F.Cu") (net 35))
 (segment (start 146.07 89.03) (end 145.1 90) (width 0.2) (layer "F.Cu") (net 42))
 (segment (start 146.07 86.2) (end 146.07 89.03) (width 0.2) (layer "F.Cu") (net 42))
 (segment (start 145.1 90) (end 141.9 90) (width 0.2) (layer "F.Cu") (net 42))
 (segment (start 147.5 90) (end 148.7 90) (width 0.2) (layer "F.Cu") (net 31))
 (segment (start 146.57 89.07) (end 147.5 90) (width 0.2) (layer "F.Cu") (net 31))
 (segment (start 146.57 86.2) (end 146.57 89.07) (width 0.2) (layer "F.Cu") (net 31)))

